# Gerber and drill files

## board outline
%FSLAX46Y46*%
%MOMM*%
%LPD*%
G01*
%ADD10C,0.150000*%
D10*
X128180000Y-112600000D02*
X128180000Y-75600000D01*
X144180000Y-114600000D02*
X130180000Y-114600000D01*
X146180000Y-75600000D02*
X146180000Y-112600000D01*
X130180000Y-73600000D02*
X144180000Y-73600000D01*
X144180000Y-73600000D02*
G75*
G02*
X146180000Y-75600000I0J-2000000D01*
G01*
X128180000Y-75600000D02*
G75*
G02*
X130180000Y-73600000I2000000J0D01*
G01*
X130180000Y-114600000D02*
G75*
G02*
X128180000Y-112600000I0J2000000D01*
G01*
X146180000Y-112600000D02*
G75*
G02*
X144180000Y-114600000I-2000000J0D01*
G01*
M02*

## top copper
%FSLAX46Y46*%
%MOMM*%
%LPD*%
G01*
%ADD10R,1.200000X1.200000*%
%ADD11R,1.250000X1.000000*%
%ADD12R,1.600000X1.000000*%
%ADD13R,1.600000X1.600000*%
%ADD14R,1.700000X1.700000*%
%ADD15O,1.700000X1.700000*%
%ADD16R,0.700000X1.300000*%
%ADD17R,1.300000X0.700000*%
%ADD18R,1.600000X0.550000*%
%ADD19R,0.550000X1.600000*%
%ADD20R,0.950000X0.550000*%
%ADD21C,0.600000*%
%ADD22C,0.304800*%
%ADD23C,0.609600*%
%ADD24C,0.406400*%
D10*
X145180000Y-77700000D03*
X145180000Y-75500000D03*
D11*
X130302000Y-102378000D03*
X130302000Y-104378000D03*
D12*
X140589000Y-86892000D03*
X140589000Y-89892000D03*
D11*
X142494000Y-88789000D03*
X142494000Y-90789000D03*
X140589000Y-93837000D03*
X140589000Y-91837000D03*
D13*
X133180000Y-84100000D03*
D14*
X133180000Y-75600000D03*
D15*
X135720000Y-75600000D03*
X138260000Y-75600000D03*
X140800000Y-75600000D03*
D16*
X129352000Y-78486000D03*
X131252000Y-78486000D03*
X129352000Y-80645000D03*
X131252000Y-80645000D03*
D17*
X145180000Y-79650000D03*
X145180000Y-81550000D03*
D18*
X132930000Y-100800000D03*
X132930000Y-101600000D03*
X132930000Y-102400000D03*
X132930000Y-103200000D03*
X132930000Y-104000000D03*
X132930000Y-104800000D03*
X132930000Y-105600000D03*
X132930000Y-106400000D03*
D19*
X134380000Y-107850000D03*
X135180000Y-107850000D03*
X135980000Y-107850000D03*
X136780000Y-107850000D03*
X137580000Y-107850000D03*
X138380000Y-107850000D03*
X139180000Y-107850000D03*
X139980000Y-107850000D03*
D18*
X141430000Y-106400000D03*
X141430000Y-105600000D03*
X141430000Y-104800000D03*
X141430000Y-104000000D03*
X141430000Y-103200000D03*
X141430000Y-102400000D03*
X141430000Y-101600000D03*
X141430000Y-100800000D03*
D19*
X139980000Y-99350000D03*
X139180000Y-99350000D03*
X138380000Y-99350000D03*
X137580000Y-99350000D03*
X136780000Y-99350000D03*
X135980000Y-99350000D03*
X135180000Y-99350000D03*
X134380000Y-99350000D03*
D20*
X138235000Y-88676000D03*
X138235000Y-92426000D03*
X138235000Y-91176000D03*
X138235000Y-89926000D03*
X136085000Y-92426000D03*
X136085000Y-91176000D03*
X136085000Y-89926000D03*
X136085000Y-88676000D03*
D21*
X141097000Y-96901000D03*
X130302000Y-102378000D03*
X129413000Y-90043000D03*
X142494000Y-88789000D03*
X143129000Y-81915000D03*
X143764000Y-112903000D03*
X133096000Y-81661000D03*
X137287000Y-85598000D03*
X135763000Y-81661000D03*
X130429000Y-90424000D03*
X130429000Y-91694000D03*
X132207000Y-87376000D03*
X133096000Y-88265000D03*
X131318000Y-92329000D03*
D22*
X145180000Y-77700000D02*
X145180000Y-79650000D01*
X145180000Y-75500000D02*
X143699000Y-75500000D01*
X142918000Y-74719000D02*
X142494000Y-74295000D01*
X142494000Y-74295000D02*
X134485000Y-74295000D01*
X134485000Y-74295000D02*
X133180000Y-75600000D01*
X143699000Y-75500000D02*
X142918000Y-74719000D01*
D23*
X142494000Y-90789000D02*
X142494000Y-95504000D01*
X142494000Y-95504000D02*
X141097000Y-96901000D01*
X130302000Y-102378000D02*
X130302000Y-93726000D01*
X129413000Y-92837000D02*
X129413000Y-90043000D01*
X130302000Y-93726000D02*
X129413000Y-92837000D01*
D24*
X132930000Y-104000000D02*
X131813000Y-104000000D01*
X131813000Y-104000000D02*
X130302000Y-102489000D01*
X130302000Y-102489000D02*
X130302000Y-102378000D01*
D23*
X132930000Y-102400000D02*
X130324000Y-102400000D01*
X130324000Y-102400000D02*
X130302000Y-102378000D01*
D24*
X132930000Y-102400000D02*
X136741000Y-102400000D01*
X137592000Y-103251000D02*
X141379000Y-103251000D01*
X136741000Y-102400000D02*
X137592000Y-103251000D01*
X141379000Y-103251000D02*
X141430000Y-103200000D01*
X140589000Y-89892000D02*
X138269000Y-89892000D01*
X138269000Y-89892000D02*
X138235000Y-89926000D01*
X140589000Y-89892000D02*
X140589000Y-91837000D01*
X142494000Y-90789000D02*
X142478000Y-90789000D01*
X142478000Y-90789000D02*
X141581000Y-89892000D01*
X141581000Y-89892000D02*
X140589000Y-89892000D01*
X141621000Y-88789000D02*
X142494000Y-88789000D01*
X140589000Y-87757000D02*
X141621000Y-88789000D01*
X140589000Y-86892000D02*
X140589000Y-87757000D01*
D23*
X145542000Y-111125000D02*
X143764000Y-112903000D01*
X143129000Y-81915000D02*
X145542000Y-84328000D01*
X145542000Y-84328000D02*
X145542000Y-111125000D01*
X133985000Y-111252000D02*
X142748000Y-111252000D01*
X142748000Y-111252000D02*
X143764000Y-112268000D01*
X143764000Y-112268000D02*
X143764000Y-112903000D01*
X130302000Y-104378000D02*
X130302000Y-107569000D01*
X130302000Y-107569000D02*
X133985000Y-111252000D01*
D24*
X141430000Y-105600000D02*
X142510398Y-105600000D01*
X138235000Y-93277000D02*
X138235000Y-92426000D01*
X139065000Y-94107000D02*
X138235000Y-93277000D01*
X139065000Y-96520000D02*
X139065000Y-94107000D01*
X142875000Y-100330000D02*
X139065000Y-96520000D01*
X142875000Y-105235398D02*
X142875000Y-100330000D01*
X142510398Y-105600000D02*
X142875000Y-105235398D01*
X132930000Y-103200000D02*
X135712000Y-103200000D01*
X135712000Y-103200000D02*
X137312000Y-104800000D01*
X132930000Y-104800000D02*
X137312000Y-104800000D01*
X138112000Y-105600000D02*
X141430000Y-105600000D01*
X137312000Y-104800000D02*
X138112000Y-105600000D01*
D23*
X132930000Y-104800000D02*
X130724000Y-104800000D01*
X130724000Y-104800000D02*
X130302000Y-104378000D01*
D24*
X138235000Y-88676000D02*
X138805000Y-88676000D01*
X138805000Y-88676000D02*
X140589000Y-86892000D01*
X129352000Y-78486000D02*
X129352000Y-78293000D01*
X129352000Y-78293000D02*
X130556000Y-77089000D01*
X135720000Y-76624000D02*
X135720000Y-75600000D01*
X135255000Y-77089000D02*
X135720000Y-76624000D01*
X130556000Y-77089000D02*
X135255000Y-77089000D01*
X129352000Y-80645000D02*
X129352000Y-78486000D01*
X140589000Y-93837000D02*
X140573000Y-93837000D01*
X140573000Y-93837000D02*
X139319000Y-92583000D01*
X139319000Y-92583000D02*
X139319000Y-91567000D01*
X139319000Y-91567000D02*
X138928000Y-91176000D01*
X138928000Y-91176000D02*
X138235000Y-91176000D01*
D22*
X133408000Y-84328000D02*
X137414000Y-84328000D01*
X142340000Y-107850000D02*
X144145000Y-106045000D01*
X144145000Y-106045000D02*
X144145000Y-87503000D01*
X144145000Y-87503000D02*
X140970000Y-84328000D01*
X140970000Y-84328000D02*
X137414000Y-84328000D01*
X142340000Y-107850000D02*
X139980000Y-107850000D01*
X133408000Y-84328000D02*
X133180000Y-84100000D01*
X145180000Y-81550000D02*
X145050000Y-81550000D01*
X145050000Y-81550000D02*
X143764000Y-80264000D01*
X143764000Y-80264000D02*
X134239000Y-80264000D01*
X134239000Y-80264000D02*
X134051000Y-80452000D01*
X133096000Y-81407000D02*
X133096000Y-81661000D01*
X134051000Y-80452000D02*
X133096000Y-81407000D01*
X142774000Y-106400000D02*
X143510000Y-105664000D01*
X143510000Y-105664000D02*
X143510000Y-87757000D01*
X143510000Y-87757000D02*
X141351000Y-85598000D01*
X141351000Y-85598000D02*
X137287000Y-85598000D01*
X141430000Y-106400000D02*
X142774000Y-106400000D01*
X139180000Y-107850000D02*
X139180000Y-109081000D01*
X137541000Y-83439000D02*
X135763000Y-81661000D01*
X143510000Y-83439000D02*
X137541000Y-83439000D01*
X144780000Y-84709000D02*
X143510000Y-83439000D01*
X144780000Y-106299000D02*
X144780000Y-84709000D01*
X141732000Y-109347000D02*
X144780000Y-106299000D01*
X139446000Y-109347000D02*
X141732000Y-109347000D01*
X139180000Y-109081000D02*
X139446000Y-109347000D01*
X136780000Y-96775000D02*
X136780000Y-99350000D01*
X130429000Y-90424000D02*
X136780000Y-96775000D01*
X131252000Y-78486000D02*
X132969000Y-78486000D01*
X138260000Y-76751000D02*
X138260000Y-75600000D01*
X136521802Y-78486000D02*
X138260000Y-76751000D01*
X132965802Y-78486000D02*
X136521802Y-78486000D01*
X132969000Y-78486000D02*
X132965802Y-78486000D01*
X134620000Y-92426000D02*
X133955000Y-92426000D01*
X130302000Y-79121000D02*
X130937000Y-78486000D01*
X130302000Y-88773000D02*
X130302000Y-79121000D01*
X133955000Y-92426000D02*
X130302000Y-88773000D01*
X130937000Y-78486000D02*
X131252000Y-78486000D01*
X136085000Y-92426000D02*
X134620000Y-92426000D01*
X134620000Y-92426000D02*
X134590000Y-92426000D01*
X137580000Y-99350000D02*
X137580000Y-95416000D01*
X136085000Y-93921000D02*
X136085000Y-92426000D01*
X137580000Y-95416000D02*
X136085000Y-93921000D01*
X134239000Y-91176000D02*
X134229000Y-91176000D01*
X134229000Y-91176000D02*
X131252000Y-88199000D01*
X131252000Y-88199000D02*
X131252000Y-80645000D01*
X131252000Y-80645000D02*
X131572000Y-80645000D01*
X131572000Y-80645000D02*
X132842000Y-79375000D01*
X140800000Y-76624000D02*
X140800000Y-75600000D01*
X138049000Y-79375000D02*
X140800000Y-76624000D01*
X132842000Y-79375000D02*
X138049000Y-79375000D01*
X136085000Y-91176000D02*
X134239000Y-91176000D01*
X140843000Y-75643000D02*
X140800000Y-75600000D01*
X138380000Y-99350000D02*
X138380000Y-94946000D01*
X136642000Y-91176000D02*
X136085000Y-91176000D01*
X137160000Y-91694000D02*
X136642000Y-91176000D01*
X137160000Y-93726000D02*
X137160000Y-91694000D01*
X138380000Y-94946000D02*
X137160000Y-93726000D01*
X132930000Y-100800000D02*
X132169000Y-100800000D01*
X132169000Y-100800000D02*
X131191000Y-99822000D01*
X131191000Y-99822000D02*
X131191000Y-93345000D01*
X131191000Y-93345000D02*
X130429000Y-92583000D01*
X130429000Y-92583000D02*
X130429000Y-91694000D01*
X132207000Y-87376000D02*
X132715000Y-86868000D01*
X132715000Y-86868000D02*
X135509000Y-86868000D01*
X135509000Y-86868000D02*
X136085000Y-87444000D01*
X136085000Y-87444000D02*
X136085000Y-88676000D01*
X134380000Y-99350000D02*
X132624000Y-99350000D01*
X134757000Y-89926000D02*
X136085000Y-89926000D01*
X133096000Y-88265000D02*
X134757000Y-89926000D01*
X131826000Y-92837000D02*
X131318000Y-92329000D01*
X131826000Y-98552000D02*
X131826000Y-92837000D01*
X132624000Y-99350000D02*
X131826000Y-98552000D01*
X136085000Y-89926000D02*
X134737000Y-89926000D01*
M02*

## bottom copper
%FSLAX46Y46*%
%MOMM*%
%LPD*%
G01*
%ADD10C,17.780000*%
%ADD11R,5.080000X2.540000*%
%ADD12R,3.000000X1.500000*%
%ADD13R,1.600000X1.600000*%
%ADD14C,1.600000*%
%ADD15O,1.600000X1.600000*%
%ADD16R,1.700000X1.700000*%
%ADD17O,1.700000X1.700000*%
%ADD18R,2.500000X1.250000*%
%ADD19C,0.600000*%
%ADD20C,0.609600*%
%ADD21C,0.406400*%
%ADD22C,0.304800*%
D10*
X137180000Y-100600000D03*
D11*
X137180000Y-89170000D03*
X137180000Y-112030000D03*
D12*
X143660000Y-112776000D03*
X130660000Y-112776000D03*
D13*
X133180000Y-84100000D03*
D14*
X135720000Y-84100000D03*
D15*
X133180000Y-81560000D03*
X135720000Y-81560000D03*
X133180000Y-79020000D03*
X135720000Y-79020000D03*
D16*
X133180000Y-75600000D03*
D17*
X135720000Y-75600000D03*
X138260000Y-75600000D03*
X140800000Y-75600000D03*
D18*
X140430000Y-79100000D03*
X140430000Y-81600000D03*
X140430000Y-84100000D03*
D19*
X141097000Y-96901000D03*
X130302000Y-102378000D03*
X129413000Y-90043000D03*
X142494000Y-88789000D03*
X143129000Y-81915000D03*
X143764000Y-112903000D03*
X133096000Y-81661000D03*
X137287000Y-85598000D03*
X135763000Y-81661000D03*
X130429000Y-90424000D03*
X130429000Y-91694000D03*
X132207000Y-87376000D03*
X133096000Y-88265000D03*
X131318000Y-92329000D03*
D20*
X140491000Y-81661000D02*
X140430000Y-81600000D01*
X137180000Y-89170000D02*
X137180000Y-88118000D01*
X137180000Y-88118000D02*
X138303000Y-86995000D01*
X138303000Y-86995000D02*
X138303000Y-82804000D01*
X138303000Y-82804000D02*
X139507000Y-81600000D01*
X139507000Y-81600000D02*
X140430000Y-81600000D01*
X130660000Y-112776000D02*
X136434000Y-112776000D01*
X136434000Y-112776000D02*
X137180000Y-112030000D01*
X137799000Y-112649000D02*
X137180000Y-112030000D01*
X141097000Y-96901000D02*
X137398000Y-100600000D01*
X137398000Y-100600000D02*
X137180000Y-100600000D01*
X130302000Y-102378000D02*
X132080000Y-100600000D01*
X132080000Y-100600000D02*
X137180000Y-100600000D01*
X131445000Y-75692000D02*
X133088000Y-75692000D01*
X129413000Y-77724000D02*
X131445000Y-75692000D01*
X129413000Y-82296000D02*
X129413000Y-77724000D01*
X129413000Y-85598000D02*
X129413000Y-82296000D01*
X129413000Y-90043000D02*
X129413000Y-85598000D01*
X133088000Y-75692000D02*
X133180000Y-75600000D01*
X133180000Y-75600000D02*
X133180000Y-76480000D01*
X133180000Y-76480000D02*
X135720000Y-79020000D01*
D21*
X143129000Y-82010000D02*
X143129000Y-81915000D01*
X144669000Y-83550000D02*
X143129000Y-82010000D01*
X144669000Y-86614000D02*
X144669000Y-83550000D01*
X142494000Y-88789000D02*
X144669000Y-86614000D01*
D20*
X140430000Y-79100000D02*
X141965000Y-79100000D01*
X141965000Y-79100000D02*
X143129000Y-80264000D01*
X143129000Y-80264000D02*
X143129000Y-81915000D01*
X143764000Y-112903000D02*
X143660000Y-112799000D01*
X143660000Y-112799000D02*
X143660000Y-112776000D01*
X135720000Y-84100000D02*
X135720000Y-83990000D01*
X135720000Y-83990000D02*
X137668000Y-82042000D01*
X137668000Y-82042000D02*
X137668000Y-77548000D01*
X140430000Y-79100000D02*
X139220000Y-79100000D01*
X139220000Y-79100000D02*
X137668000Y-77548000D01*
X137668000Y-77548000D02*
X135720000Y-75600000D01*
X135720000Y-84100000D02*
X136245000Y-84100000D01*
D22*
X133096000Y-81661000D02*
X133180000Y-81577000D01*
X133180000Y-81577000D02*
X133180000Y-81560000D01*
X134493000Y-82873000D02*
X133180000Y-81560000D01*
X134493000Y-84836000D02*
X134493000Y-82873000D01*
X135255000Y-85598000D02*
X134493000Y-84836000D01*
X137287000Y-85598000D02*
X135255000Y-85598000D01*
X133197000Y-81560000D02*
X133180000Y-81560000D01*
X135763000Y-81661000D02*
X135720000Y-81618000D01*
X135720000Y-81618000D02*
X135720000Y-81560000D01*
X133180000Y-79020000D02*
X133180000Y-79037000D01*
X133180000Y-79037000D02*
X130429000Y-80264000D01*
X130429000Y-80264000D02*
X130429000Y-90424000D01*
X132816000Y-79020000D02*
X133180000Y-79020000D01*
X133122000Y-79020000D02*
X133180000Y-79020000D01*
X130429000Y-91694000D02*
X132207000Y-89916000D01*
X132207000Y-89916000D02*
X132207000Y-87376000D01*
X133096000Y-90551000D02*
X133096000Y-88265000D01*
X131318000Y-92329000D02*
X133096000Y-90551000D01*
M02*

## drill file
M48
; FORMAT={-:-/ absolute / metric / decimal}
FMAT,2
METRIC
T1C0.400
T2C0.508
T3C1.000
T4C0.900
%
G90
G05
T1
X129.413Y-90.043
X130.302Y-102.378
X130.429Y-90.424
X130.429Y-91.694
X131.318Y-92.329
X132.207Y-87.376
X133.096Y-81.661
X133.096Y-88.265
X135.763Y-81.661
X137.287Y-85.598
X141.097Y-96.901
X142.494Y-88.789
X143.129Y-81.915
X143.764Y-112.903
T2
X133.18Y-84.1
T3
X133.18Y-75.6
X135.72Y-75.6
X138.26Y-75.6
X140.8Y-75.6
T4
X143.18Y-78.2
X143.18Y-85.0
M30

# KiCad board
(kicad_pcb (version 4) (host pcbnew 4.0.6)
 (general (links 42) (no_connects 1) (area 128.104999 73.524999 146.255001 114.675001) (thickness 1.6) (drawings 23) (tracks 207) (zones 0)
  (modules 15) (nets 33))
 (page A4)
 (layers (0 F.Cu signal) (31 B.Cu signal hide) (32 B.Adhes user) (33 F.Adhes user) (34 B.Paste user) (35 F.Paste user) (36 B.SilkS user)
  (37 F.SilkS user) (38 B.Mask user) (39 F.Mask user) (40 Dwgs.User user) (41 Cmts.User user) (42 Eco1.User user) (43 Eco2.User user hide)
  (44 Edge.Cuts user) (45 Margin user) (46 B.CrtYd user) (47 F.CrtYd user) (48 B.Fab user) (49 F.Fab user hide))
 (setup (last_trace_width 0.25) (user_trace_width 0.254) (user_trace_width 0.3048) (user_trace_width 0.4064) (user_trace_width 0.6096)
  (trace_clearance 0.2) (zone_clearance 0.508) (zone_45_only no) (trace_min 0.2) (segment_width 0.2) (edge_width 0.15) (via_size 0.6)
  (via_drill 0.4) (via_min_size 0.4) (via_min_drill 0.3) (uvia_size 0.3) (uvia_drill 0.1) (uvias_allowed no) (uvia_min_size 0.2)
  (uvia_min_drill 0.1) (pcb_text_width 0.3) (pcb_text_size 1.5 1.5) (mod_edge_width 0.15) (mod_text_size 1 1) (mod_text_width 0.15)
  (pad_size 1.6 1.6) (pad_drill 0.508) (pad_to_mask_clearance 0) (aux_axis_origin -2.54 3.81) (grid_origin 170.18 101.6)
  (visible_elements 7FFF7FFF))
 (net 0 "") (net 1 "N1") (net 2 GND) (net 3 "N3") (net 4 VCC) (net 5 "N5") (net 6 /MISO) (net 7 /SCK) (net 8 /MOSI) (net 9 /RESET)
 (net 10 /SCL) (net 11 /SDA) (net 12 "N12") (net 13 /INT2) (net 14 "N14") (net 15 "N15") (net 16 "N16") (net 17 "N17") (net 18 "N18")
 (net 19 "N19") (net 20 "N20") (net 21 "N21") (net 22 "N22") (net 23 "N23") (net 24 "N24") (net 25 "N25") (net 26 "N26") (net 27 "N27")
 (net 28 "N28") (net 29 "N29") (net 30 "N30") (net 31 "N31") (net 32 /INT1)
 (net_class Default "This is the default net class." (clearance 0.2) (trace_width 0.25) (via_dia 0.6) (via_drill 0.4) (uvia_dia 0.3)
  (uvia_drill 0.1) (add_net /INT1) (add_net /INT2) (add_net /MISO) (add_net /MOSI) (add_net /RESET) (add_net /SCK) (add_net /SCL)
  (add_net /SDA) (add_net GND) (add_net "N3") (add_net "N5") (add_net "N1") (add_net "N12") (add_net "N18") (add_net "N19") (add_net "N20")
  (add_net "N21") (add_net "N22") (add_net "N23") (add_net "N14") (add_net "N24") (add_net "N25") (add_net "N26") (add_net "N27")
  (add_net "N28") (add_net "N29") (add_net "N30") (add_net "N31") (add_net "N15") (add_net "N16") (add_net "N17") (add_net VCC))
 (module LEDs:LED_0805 (layer F.Cu) (at 145.18 76.6 270)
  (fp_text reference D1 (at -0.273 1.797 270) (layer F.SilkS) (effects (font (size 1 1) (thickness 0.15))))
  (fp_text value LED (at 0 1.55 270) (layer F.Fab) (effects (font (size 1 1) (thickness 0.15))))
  (pad 2 smd rect (at 1.1 0 90) (size 1.2 1.2) (layers F.Cu F.Paste F.Mask) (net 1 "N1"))
  (pad 1 smd rect (at -1.1 0 90) (size 1.2 1.2) (layers F.Cu F.Paste F.Mask) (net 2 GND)))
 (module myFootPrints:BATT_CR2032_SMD (layer B.Cu) (at 137.18 100.6 270)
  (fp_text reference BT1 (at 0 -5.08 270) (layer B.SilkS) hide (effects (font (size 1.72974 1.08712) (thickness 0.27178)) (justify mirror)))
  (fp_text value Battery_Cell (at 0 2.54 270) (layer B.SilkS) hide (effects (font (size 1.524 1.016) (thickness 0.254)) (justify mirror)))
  (pad 2 smd circle (at 0 0 270) (size 17.78 17.78) (layers B.Cu B.Paste B.Mask) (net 2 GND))
  (pad 1 smd rect (at -11.43 0 270) (size 2.54 5.08) (layers B.Cu B.Paste B.Mask) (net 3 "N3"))
  (pad 1 smd rect (at 11.43 0 270) (size 2.54 5.08) (layers B.Cu B.Paste B.Mask) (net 3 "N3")))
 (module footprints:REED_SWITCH (layer B.Cu) (at 137.16 112.776 180)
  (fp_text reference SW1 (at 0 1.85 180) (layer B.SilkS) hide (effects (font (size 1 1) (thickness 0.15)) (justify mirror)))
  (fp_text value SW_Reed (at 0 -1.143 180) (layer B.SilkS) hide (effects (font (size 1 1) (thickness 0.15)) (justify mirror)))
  (pad 1 smd rect (at -6.5 0 180) (size 3 1.5) (layers B.Cu B.Paste B.Mask) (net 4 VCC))
  (pad 2 smd rect (at 6.5 0 180) (size 3 1.5) (layers B.Cu B.Paste B.Mask) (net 3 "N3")))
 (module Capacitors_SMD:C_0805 (layer F.Cu) (at 130.302 103.378 270)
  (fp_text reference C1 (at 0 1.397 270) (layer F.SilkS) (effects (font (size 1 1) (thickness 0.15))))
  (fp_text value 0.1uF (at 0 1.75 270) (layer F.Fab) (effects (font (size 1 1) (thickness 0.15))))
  (pad 1 smd rect (at -1 0 270) (size 1 1.25) (layers F.Cu F.Paste F.Mask) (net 2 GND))
  (pad 2 smd rect (at 1 0 270) (size 1 1.25) (layers F.Cu F.Paste F.Mask) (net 4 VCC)))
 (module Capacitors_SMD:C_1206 (layer F.Cu) (at 140.589 88.392 270)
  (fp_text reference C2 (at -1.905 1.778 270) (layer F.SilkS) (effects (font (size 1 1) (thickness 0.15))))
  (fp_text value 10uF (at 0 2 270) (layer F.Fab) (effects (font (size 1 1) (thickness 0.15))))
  (pad 1 smd rect (at -1.5 0 270) (size 1 1.6) (layers F.Cu F.Paste F.Mask) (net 4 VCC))
  (pad 2 smd rect (at 1.5 0 270) (size 1 1.6) (layers F.Cu F.Paste F.Mask) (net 2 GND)))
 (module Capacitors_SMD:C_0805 (layer F.Cu) (at 142.494 89.789 270)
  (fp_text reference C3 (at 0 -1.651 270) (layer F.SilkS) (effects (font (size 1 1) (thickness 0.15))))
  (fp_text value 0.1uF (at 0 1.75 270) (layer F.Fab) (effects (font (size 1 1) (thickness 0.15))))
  (pad 1 smd rect (at -1 0 270) (size 1 1.25) (layers F.Cu F.Paste F.Mask) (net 4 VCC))
  (pad 2 smd rect (at 1 0 270) (size 1 1.25) (layers F.Cu F.Paste F.Mask) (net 2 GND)))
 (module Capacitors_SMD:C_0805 (layer F.Cu) (at 140.589 92.837 90)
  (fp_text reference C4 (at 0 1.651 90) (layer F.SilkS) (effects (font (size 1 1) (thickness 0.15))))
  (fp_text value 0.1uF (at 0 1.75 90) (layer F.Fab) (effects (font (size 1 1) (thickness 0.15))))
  (pad 1 smd rect (at -1 0 90) (size 1 1.25) (layers F.Cu F.Paste F.Mask) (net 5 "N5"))
  (pad 2 smd rect (at 1 0 90) (size 1 1.25) (layers F.Cu F.Paste F.Mask) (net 2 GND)))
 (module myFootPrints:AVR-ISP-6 (layer B.Cu) (at 133.18 84.1)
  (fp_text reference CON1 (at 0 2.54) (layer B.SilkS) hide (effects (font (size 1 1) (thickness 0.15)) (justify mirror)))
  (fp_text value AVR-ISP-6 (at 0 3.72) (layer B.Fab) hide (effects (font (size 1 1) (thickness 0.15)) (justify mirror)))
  (pad 1 thru_hole rect (at 0 0) (size 1.6 1.6) (drill 0.508) (layers *.Cu B.Mask) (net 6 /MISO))
  (pad 2 smd circle (at 2.54 0) (size 1.6 1.6) (layers B.Cu B.Paste B.Mask) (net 4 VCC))
  (pad 3 smd oval (at 0 -2.54) (size 1.6 1.6) (layers B.Cu B.Paste B.Mask) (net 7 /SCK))
  (pad 4 smd oval (at 2.54 -2.54) (size 1.6 1.6) (layers B.Cu B.Paste B.Mask) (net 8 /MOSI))
  (pad 5 smd oval (at 0 -5.08) (size 1.6 1.6) (layers B.Cu B.Paste B.Mask) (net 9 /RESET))
  (pad 6 smd oval (at 2.54 -5.08) (size 1.6 1.6) (layers B.Cu B.Paste B.Mask) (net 2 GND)))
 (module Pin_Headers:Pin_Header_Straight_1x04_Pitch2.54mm (layer F.Cu) (at 133.18 75.6 90)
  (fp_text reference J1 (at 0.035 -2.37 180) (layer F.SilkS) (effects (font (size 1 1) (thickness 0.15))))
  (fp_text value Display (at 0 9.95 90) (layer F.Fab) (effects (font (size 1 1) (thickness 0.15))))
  (pad 1 thru_hole rect (at 0 0 90) (size 1.7 1.7) (drill 1) (layers *.Cu *.Mask) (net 2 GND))
  (pad 2 thru_hole oval (at 0 2.54 90) (size 1.7 1.7) (drill 1) (layers *.Cu *.Mask) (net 4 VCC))
  (pad 3 thru_hole oval (at 0 5.08 90) (size 1.7 1.7) (drill 1) (layers *.Cu *.Mask) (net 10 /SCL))
  (pad 4 thru_hole oval (at 0 7.62 90) (size 1.7 1.7) (drill 1) (layers *.Cu *.Mask) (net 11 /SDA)))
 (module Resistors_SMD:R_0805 (layer F.Cu) (at 130.302 78.486)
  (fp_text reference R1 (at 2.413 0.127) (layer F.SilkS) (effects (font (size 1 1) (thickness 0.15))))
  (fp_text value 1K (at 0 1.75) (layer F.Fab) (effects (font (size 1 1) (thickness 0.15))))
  (pad 1 smd rect (at -0.95 0) (size 0.7 1.3) (layers F.Cu F.Paste F.Mask) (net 4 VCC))
  (pad 2 smd rect (at 0.95 0) (size 0.7 1.3) (layers F.Cu F.Paste F.Mask) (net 10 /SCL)))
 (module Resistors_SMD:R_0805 (layer F.Cu) (at 130.302 80.645)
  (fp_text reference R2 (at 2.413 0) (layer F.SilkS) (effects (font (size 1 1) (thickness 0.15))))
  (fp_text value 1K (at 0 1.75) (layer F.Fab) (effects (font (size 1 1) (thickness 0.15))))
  (pad 1 smd rect (at -0.95 0) (size 0.7 1.3) (layers F.Cu F.Paste F.Mask) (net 4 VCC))
  (pad 2 smd rect (at 0.95 0) (size 0.7 1.3) (layers F.Cu F.Paste F.Mask) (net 11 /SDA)))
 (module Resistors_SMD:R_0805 (layer F.Cu) (at 145.18 80.6 270)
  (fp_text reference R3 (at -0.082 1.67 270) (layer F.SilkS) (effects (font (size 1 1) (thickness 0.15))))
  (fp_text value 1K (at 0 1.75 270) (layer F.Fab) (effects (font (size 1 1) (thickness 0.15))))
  (pad 1 smd rect (at -0.95 0 270) (size 0.7 1.3) (layers F.Cu F.Paste F.Mask) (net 1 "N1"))
  (pad 2 smd rect (at 0.95 0 270) (size 0.7 1.3) (layers F.Cu F.Paste F.Mask) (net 7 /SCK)))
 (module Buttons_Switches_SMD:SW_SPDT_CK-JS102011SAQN (layer B.Cu) (at 143.18 81.6 270)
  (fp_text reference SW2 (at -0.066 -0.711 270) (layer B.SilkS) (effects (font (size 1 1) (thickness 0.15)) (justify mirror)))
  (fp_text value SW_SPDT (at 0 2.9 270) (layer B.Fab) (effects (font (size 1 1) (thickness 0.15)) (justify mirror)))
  (pad 1 smd rect (at -2.5 2.75 270) (size 1.25 2.5) (layers B.Cu B.Paste B.Mask) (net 4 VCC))
  (pad 2 smd rect (at 0 2.75 270) (size 1.25 2.5) (layers B.Cu B.Paste B.Mask) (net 3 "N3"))
  (pad 3 smd rect (at 2.5 2.75 270) (size 1.25 2.5) (layers B.Cu B.Paste B.Mask) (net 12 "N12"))
  (pad "" np_thru_hole circle (at -3.4 0 270) (size 0.9 0.9) (drill 0.9) (layers *.Cu *.Mask))
  (pad "" np_thru_hole circle (at 3.4 0 270) (size 0.9 0.9) (drill 0.9) (layers *.Cu *.Mask)))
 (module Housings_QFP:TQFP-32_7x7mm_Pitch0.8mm (layer F.Cu) (at 137.18 103.6)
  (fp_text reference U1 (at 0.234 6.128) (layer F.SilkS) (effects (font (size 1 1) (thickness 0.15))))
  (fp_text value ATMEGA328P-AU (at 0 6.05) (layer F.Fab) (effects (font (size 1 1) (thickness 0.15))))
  (pad 1 smd rect (at -4.25 -2.8) (size 1.6 0.55) (layers F.Cu F.Paste F.Mask) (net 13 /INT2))
  (pad 2 smd rect (at -4.25 -2) (size 1.6 0.55) (layers F.Cu F.Paste F.Mask) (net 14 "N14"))
  (pad 3 smd rect (at -4.25 -1.2) (size 1.6 0.55) (layers F.Cu F.Paste F.Mask) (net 2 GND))
  (pad 4 smd rect (at -4.25 -0.4) (size 1.6 0.55) (layers F.Cu F.Paste F.Mask) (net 4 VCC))
  (pad 5 smd rect (at -4.25 0.4) (size 1.6 0.55) (layers F.Cu F.Paste F.Mask) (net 2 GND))
  (pad 6 smd rect (at -4.25 1.2) (size 1.6 0.55) (layers F.Cu F.Paste F.Mask) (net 4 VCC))
  (pad 7 smd rect (at -4.25 2) (size 1.6 0.55) (layers F.Cu F.Paste F.Mask) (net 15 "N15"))
  (pad 8 smd rect (at -4.25 2.8) (size 1.6 0.55) (layers F.Cu F.Paste F.Mask) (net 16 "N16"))
  (pad 9 smd rect (at -2.8 4.25 90) (size 1.6 0.55) (layers F.Cu F.Paste F.Mask) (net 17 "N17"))
  (pad 10 smd rect (at -2 4.25 90) (size 1.6 0.55) (layers F.Cu F.Paste F.Mask) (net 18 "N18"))
  (pad 11 smd rect (at -1.2 4.25 90) (size 1.6 0.55) (layers F.Cu F.Paste F.Mask) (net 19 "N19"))
  (pad 12 smd rect (at -0.4 4.25 90) (size 1.6 0.55) (layers F.Cu F.Paste F.Mask) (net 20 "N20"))
  (pad 13 smd rect (at 0.4 4.25 90) (size 1.6 0.55) (layers F.Cu F.Paste F.Mask) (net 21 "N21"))
  (pad 14 smd rect (at 1.2 4.25 90) (size 1.6 0.55) (layers F.Cu F.Paste F.Mask) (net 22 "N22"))
  (pad 15 smd rect (at 2 4.25 90) (size 1.6 0.55) (layers F.Cu F.Paste F.Mask) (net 8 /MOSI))
  (pad 16 smd rect (at 2.8 4.25 90) (size 1.6 0.55) (layers F.Cu F.Paste F.Mask) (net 6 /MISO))
  (pad 17 smd rect (at 4.25 2.8) (size 1.6 0.55) (layers F.Cu F.Paste F.Mask) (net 7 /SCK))
  (pad 18 smd rect (at 4.25 2) (size 1.6 0.55) (layers F.Cu F.Paste F.Mask) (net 4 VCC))
  (pad 19 smd rect (at 4.25 1.2) (size 1.6 0.55) (layers F.Cu F.Paste F.Mask) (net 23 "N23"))
  (pad 20 smd rect (at 4.25 0.4) (size 1.6 0.55) (layers F.Cu F.Paste F.Mask) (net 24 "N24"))
  (pad 21 smd rect (at 4.25 -0.4) (size 1.6 0.55) (layers F.Cu F.Paste F.Mask) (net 2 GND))
  (pad 22 smd rect (at 4.25 -1.2) (size 1.6 0.55) (layers F.Cu F.Paste F.Mask) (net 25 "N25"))
  (pad 23 smd rect (at 4.25 -2) (size 1.6 0.55) (layers F.Cu F.Paste F.Mask) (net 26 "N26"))
  (pad 24 smd rect (at 4.25 -2.8) (size 1.6 0.55) (layers F.Cu F.Paste F.Mask) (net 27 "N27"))
  (pad 25 smd rect (at 2.8 -4.25 90) (size 1.6 0.55) (layers F.Cu F.Paste F.Mask) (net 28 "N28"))
  (pad 26 smd rect (at 2 -4.25 90) (size 1.6 0.55) (layers F.Cu F.Paste F.Mask) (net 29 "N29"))
  (pad 27 smd rect (at 1.2 -4.25 90) (size 1.6 0.55) (layers F.Cu F.Paste F.Mask) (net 11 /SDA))
  (pad 28 smd rect (at 0.4 -4.25 90) (size 1.6 0.55) (layers F.Cu F.Paste F.Mask) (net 10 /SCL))
  (pad 29 smd rect (at -0.4 -4.25 90) (size 1.6 0.55) (layers F.Cu F.Paste F.Mask) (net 9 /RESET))
  (pad 30 smd rect (at -1.2 -4.25 90) (size 1.6 0.55) (layers F.Cu F.Paste F.Mask) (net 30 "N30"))
  (pad 31 smd rect (at -2 -4.25 90) (size 1.6 0.55) (layers F.Cu F.Paste F.Mask) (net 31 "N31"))
  (pad 32 smd rect (at -2.8 -4.25 90) (size 1.6 0.55) (layers F.Cu F.Paste F.Mask) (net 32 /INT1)))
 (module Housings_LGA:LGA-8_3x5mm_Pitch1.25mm (layer F.Cu) (at 137.16 90.551 180)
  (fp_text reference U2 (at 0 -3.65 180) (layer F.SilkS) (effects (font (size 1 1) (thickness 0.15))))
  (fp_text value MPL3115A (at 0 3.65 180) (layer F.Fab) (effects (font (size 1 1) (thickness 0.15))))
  (pad 4 smd rect (at -1.075 1.875 180) (size 0.95 0.55) (layers F.Cu F.Paste F.Mask) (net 4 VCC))
  (pad 1 smd rect (at -1.075 -1.875 180) (size 0.95 0.55) (layers F.Cu F.Paste F.Mask) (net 4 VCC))
  (pad 2 smd rect (at -1.075 -0.625 180) (size 0.95 0.55) (layers F.Cu F.Paste F.Mask) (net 5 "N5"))
  (pad 3 smd rect (at -1.075 0.625 180) (size 0.95 0.55) (layers F.Cu F.Paste F.Mask) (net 2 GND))
  (pad 8 smd rect (at 1.075 -1.875 180) (size 0.95 0.55) (layers F.Cu F.Paste F.Mask) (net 10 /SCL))
  (pad 7 smd rect (at 1.075 -0.625 180) (size 0.95 0.55) (layers F.Cu F.Paste F.Mask) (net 11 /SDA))
  (pad 6 smd rect (at 1.075 0.625 180) (size 0.95 0.55) (layers F.Cu F.Paste F.Mask) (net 32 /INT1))
  (pad 5 smd rect (at 1.075 1.875 180) (size 0.95 0.55) (layers F.Cu F.Paste F.Mask) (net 13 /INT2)))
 (gr_line (start 128.18 112.6) (end 128.18 75.6) (angle 90) (layer Edge.Cuts) (width 0.15))
 (gr_line (start 144.18 114.6) (end 130.18 114.6) (angle 90) (layer Edge.Cuts) (width 0.15))
 (gr_line (start 146.18 75.6) (end 146.18 112.6) (angle 90) (layer Edge.Cuts) (width 0.15))
 (gr_line (start 130.18 73.6) (end 144.18 73.6) (angle 90) (layer Edge.Cuts) (width 0.15))
 (gr_arc (start 144.18 75.6) (end 144.18 73.6) (angle 90) (layer Edge.Cuts) (width 0.15))
 (gr_arc (start 130.18 75.6) (end 128.18 75.6) (angle 90) (layer Edge.Cuts) (width 0.15))
 (gr_arc (start 130.18 112.6) (end 130.18 114.6) (angle 90) (layer Edge.Cuts) (width 0.15))
 (gr_arc (start 144.18 112.6) (end 146.18 112.6) (angle 90) (layer Edge.Cuts) (width 0.15))
 (segment (start 140.491 81.661) (end 140.43 81.6) (width 0.6096) (layer B.Cu) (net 3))
 (segment (start 137.18 89.17) (end 137.18 88.118) (width 0.6096) (layer B.Cu) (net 3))
 (segment (start 137.18 88.118) (end 138.303 86.995) (width 0.6096) (layer B.Cu) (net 3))
 (segment (start 138.303 86.995) (end 138.303 82.804) (width 0.6096) (layer B.Cu) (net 3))
 (segment (start 138.303 82.804) (end 139.507 81.6) (width 0.6096) (layer B.Cu) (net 3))
 (segment (start 139.507 81.6) (end 140.43 81.6) (width 0.6096) (layer B.Cu) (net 3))
 (segment (start 130.66 112.776) (end 136.434 112.776) (width 0.6096) (layer B.Cu) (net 3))
 (segment (start 136.434 112.776) (end 137.18 112.03) (width 0.6096) (layer B.Cu) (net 3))
 (segment (start 137.799 112.649) (end 137.18 112.03) (width 0.6096) (layer B.Cu) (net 3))
 (segment (start 145.18 77.7) (end 145.18 79.65) (width 0.3048) (layer F.Cu) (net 1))
 (segment (start 145.18 75.5) (end 143.699 75.5) (width 0.3048) (layer F.Cu) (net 2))
 (segment (start 142.918 74.719) (end 142.494 74.295) (width 0.3048) (layer F.Cu) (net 2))
 (segment (start 142.494 74.295) (end 134.485 74.295) (width 0.3048) (layer F.Cu) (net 2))
 (segment (start 134.485 74.295) (end 133.18 75.6) (width 0.3048) (layer F.Cu) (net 2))
 (segment (start 143.699 75.5) (end 142.918 74.719) (width 0.3048) (layer F.Cu) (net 2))
 (segment (start 142.494 90.789) (end 142.494 95.504) (width 0.6096) (layer F.Cu) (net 2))
 (segment (start 141.097 96.901) (end 137.398 100.6) (width 0.6096) (layer B.Cu) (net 2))
 (via (at 141.097 96.901) (size 0.6) (drill 0.4) (layers F.Cu B.Cu) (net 2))
 (segment (start 142.494 95.504) (end 141.097 96.901) (width 0.6096) (layer F.Cu) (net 2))
 (segment (start 137.398 100.6) (end 137.18 100.6) (width 0.6096) (layer B.Cu) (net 2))
 (via (at 130.302 102.378) (size 0.6) (drill 0.4) (layers F.Cu B.Cu) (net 2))
 (segment (start 130.302 102.378) (end 132.08 100.6) (width 0.6096) (layer B.Cu) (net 2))
 (segment (start 132.08 100.6) (end 137.18 100.6) (width 0.6096) (layer B.Cu) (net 2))
 (segment (start 130.302 102.378) (end 130.302 93.726) (width 0.6096) (layer F.Cu) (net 2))
 (segment (start 131.445 75.692) (end 133.088 75.692) (width 0.6096) (layer B.Cu) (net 2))
 (segment (start 129.413 77.724) (end 131.445 75.692) (width 0.6096) (layer B.Cu) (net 2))
 (segment (start 129.413 82.296) (end 129.413 77.724) (width 0.6096) (layer B.Cu) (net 2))
 (segment (start 129.413 85.598) (end 129.413 82.296) (width 0.6096) (layer B.Cu) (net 2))
 (segment (start 129.413 90.043) (end 129.413 85.598) (width 0.6096) (layer B.Cu) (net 2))
 (via (at 129.413 90.043) (size 0.6) (drill 0.4) (layers F.Cu B.Cu) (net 2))
 (segment (start 129.413 92.837) (end 129.413 90.043) (width 0.6096) (layer F.Cu) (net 2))
 (segment (start 130.302 93.726) (end 129.413 92.837) (width 0.6096) (layer F.Cu) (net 2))
 (segment (start 133.088 75.692) (end 133.18 75.6) (width 0.6096) (layer B.Cu) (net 2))
 (segment (start 132.93 104) (end 131.813 104) (width 0.4064) (layer F.Cu) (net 2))
 (segment (start 131.813 104) (end 130.302 102.489) (width 0.4064) (layer F.Cu) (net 2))
 (segment (start 130.302 102.489) (end 130.302 102.378) (width 0.4064) (layer F.Cu) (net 2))
 (segment (start 132.93 102.4) (end 130.324 102.4) (width 0.6096) (layer F.Cu) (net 2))
 (segment (start 130.324 102.4) (end 130.302 102.378) (width 0.6096) (layer F.Cu) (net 2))
 (segment (start 132.93 102.4) (end 136.741 102.4) (width 0.4064) (layer F.Cu) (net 2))
 (segment (start 137.592 103.251) (end 141.379 103.251) (width 0.4064) (layer F.Cu) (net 2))
 (segment (start 136.741 102.4) (end 137.592 103.251) (width 0.4064) (layer F.Cu) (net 2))
 (segment (start 141.379 103.251) (end 141.43 103.2) (width 0.4064) (layer F.Cu) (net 2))
 (segment (start 140.589 89.892) (end 138.269 89.892) (width 0.4064) (layer F.Cu) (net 2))
 (segment (start 138.269 89.892) (end 138.235 89.926) (width 0.4064) (layer F.Cu) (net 2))
 (segment (start 140.589 89.892) (end 140.589 91.837) (width 0.4064) (layer F.Cu) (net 2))
 (segment (start 142.494 90.789) (end 142.478 90.789) (width 0.4064) (layer F.Cu) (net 2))
 (segment (start 142.478 90.789) (end 141.581 89.892) (width 0.4064) (layer F.Cu) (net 2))
 (segment (start 141.581 89.892) (end 140.589 89.892) (width 0.4064) (layer F.Cu) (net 2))
 (segment (start 133.18 75.6) (end 133.18 76.48) (width 0.6096) (layer B.Cu) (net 2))
 (segment (start 133.18 76.48) (end 135.72 79.02) (width 0.6096) (layer B.Cu) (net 2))
 (via (at 142.494 88.789) (size 0.6) (drill 0.4) (layers F.Cu B.Cu) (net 4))
 (segment (start 141.621 88.789) (end 142.494 88.789) (width 0.4064) (layer F.Cu) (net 4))
 (segment (start 140.589 87.757) (end 141.621 88.789) (width 0.4064) (layer F.Cu) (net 4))
 (segment (start 140.589 86.892) (end 140.589 87.757) (width 0.4064) (layer F.Cu) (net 4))
 (segment (start 143.129 82.01) (end 143.129 81.915) (width 0.4064) (layer B.Cu) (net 4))
 (segment (start 144.669 83.55) (end 143.129 82.01) (width 0.4064) (layer B.Cu) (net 4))
 (segment (start 144.669 86.614) (end 144.669 83.55) (width 0.4064) (layer B.Cu) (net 4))
 (segment (start 142.494 88.789) (end 144.669 86.614) (width 0.4064) (layer B.Cu) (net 4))
 (segment (start 140.43 79.1) (end 141.965 79.1) (width 0.6096) (layer B.Cu) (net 4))
 (segment (start 141.965 79.1) (end 143.129 80.264) (width 0.6096) (layer B.Cu) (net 4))
 (segment (start 143.129 80.264) (end 143.129 81.915) (width 0.6096) (layer B.Cu) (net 4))
 (segment (start 145.542 111.125) (end 143.764 112.903) (width 0.6096) (layer F.Cu) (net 4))
 (via (at 143.129 81.915) (size 0.6) (drill 0.4) (layers F.Cu B.Cu) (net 4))
 (segment (start 143.129 81.915) (end 145.542 84.328) (width 0.6096) (layer F.Cu) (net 4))
 (segment (start 145.542 84.328) (end 145.542 111.125) (width 0.6096) (layer F.Cu) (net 4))
 (segment (start 133.985 111.252) (end 142.748 111.252) (width 0.6096) (layer F.Cu) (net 4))
 (segment (start 142.748 111.252) (end 143.764 112.268) (width 0.6096) (layer F.Cu) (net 4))
 (segment (start 143.764 112.268) (end 143.764 112.903) (width 0.6096) (layer F.Cu) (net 4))
 (segment (start 130.302 104.378) (end 130.302 107.569) (width 0.6096) (layer F.Cu) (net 4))
 (segment (start 130.302 107.569) (end 133.985 111.252) (width 0.6096) (layer F.Cu) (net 4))
 (segment (start 143.764 112.903) (end 143.66 112.799) (width 0.6096) (layer B.Cu) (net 4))
 (via (at 143.764 112.903) (size 0.6) (drill 0.4) (layers F.Cu B.Cu) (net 4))
 (segment (start 143.66 112.799) (end 143.66 112.776) (width 0.6096) (layer B.Cu) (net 4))
 (segment (start 135.72 84.1) (end 135.72 83.99) (width 0.6096) (layer B.Cu) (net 4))
 (segment (start 135.72 83.99) (end 137.668 82.042) (width 0.6096) (layer B.Cu) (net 4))
 (segment (start 137.668 82.042) (end 137.668 77.548) (width 0.6096) (layer B.Cu) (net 4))
 (segment (start 140.43 79.1) (end 139.22 79.1) (width 0.6096) (layer B.Cu) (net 4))
 (segment (start 139.22 79.1) (end 137.668 77.548) (width 0.6096) (layer B.Cu) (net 4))
 (segment (start 137.668 77.548) (end 135.72 75.6) (width 0.6096) (layer B.Cu) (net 4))
 (segment (start 141.43 105.6) (end 142.510398 105.6) (width 0.4064) (layer F.Cu) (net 4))
 (segment (start 138.235 93.277) (end 138.235 92.426) (width 0.4064) (layer F.Cu) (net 4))
 (segment (start 139.065 94.107) (end 138.235 93.277) (width 0.4064) (layer F.Cu) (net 4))
 (segment (start 139.065 96.52) (end 139.065 94.107) (width 0.4064) (layer F.Cu) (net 4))
 (segment (start 142.875 100.33) (end 139.065 96.52) (width 0.4064) (layer F.Cu) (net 4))
 (segment (start 142.875 105.235398) (end 142.875 100.33) (width 0.4064) (layer F.Cu) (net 4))
 (segment (start 142.510398 105.6) (end 142.875 105.235398) (width 0.4064) (layer F.Cu) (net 4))
 (segment (start 132.93 103.2) (end 135.712 103.2) (width 0.4064) (layer F.Cu) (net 4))
 (segment (start 135.712 103.2) (end 137.312 104.8) (width 0.4064) (layer F.Cu) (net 4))
 (segment (start 132.93 104.8) (end 137.312 104.8) (width 0.4064) (layer F.Cu) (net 4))
 (segment (start 138.112 105.6) (end 141.43 105.6) (width 0.4064) (layer F.Cu) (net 4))
 (segment (start 137.312 104.8) (end 138.112 105.6) (width 0.4064) (layer F.Cu) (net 4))
 (segment (start 132.93 104.8) (end 130.724 104.8) (width 0.6096) (layer F.Cu) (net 4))
 (segment (start 130.724 104.8) (end 130.302 104.378) (width 0.6096) (layer F.Cu) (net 4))
 (segment (start 138.235 88.676) (end 138.805 88.676) (width 0.4064) (layer F.Cu) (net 4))
 (segment (start 138.805 88.676) (end 140.589 86.892) (width 0.4064) (layer F.Cu) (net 4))
 (segment (start 129.352 78.486) (end 129.352 78.293) (width 0.4064) (layer F.Cu) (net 4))
 (segment (start 129.352 78.293) (end 130.556 77.089) (width 0.4064) (layer F.Cu) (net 4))
 (segment (start 135.72 76.624) (end 135.72 75.6) (width 0.4064) (layer F.Cu) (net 4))
 (segment (start 135.255 77.089) (end 135.72 76.624) (width 0.4064) (layer F.Cu) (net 4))
 (segment (start 130.556 77.089) (end 135.255 77.089) (width 0.4064) (layer F.Cu) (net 4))
 (segment (start 129.352 80.645) (end 129.352 78.486) (width 0.4064) (layer F.Cu) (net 4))
 (segment (start 135.72 84.1) (end 136.245 84.1) (width 0.6096) (layer B.Cu) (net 4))
 (segment (start 140.589 93.837) (end 140.573 93.837) (width 0.4064) (layer F.Cu) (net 5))
 (segment (start 140.573 93.837) (end 139.319 92.583) (width 0.4064) (layer F.Cu) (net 5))
 (segment (start 139.319 92.583) (end 139.319 91.567) (width 0.4064) (layer F.Cu) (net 5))
 (segment (start 139.319 91.567) (end 138.928 91.176) (width 0.4064) (layer F.Cu) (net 5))
 (segment (start 138.928 91.176) (end 138.235 91.176) (width 0.4064) (layer F.Cu) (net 5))
 (segment (start 133.408 84.328) (end 137.414 84.328) (width 0.3048) (layer F.Cu) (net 6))
 (segment (start 142.34 107.85) (end 144.145 106.045) (width 0.3048) (layer F.Cu) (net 6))
 (segment (start 144.145 106.045) (end 144.145 87.503) (width 0.3048) (layer F.Cu) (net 6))
 (segment (start 144.145 87.503) (end 140.97 84.328) (width 0.3048) (layer F.Cu) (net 6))
 (segment (start 140.97 84.328) (end 137.414 84.328) (width 0.3048) (layer F.Cu) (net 6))
 (segment (start 142.34 107.85) (end 139.98 107.85) (width 0.3048) (layer F.Cu) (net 6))
 (segment (start 133.408 84.328) (end 133.18 84.1) (width 0.3048) (layer F.Cu) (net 6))
 (segment (start 145.18 81.55) (end 145.05 81.55) (width 0.3048) (layer F.Cu) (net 7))
 (segment (start 145.05 81.55) (end 143.764 80.264) (width 0.3048) (layer F.Cu) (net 7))
 (segment (start 143.764 80.264) (end 134.239 80.264) (width 0.3048) (layer F.Cu) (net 7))
 (segment (start 134.239 80.264) (end 134.051 80.452) (width 0.3048) (layer F.Cu) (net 7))
 (segment (start 133.096 81.661) (end 133.18 81.577) (width 0.3048) (layer B.Cu) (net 7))
 (via (at 133.096 81.661) (size 0.6) (drill 0.4) (layers F.Cu B.Cu) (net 7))
 (segment (start 133.096 81.407) (end 133.096 81.661) (width 0.3048) (layer F.Cu) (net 7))
 (segment (start 134.051 80.452) (end 133.096 81.407) (width 0.3048) (layer F.Cu) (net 7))
 (segment (start 133.18 81.577) (end 133.18 81.56) (width 0.3048) (layer B.Cu) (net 7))
 (via (at 137.287 85.598) (size 0.6) (drill 0.4) (layers F.Cu B.Cu) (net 7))
 (segment (start 142.774 106.4) (end 143.51 105.664) (width 0.3048) (layer F.Cu) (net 7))
 (segment (start 143.51 105.664) (end 143.51 87.757) (width 0.3048) (layer F.Cu) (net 7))
 (segment (start 143.51 87.757) (end 141.351 85.598) (width 0.3048) (layer F.Cu) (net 7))
 (segment (start 141.351 85.598) (end 137.287 85.598) (width 0.3048) (layer F.Cu) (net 7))
 (segment (start 141.43 106.4) (end 142.774 106.4) (width 0.3048) (layer F.Cu) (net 7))
 (segment (start 134.493 82.873) (end 133.18 81.56) (width 0.3048) (layer B.Cu) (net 7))
 (segment (start 134.493 84.836) (end 134.493 82.873) (width 0.3048) (layer B.Cu) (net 7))
 (segment (start 135.255 85.598) (end 134.493 84.836) (width 0.3048) (layer B.Cu) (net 7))
 (segment (start 137.287 85.598) (end 135.255 85.598) (width 0.3048) (layer B.Cu) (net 7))
 (segment (start 133.197 81.56) (end 133.18 81.56) (width 0.3048) (layer B.Cu) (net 7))
 (segment (start 139.18 107.85) (end 139.18 109.081) (width 0.3048) (layer F.Cu) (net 8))
 (segment (start 135.763 81.661) (end 135.72 81.618) (width 0.3048) (layer B.Cu) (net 8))
 (via (at 135.763 81.661) (size 0.6) (drill 0.4) (layers F.Cu B.Cu) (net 8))
 (segment (start 137.541 83.439) (end 135.763 81.661) (width 0.3048) (layer F.Cu) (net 8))
 (segment (start 143.51 83.439) (end 137.541 83.439) (width 0.3048) (layer F.Cu) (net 8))
 (segment (start 144.78 84.709) (end 143.51 83.439) (width 0.3048) (layer F.Cu) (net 8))
 (segment (start 144.78 106.299) (end 144.78 84.709) (width 0.3048) (layer F.Cu) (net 8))
 (segment (start 141.732 109.347) (end 144.78 106.299) (width 0.3048) (layer F.Cu) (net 8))
 (segment (start 139.446 109.347) (end 141.732 109.347) (width 0.3048) (layer F.Cu) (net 8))
 (segment (start 139.18 109.081) (end 139.446 109.347) (width 0.3048) (layer F.Cu) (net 8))
 (segment (start 135.72 81.618) (end 135.72 81.56) (width 0.3048) (layer B.Cu) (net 8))
 (segment (start 133.18 79.02) (end 133.18 79.037) (width 0.3048) (layer B.Cu) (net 9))
 (segment (start 133.18 79.037) (end 130.429 80.264) (width 0.3048) (layer B.Cu) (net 9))
 (segment (start 136.78 96.775) (end 136.78 99.35) (width 0.3048) (layer F.Cu) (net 9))
 (segment (start 130.429 90.424) (end 136.78 96.775) (width 0.3048) (layer F.Cu) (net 9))
 (via (at 130.429 90.424) (size 0.6) (drill 0.4) (layers F.Cu B.Cu) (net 9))
 (segment (start 130.429 80.264) (end 130.429 90.424) (width 0.3048) (layer B.Cu) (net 9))
 (segment (start 132.816 79.02) (end 133.18 79.02) (width 0.3048) (layer B.Cu) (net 9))
 (segment (start 133.122 79.02) (end 133.18 79.02) (width 0.3048) (layer B.Cu) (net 9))
 (segment (start 131.252 78.486) (end 132.969 78.486) (width 0.3048) (layer F.Cu) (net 10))
 (segment (start 138.26 76.751) (end 138.26 75.6) (width 0.3048) (layer F.Cu) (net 10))
 (segment (start 136.521802 78.486) (end 138.26 76.751) (width 0.3048) (layer F.Cu) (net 10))
 (segment (start 132.965802 78.486) (end 136.521802 78.486) (width 0.3048) (layer F.Cu) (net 10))
 (segment (start 132.969 78.486) (end 132.965802 78.486) (width 0.3048) (layer F.Cu) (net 10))
 (segment (start 134.62 92.426) (end 133.955 92.426) (width 0.3048) (layer F.Cu) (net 10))
 (segment (start 130.302 79.121) (end 130.937 78.486) (width 0.3048) (layer F.Cu) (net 10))
 (segment (start 130.302 88.773) (end 130.302 79.121) (width 0.3048) (layer F.Cu) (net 10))
 (segment (start 133.955 92.426) (end 130.302 88.773) (width 0.3048) (layer F.Cu) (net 10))
 (segment (start 130.937 78.486) (end 131.252 78.486) (width 0.3048) (layer F.Cu) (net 10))
 (segment (start 136.085 92.426) (end 134.62 92.426) (width 0.3048) (layer F.Cu) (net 10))
 (segment (start 134.62 92.426) (end 134.59 92.426) (width 0.3048) (layer F.Cu) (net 10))
 (segment (start 137.58 99.35) (end 137.58 95.416) (width 0.3048) (layer F.Cu) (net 10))
 (segment (start 136.085 93.921) (end 136.085 92.426) (width 0.3048) (layer F.Cu) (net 10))
 (segment (start 137.58 95.416) (end 136.085 93.921) (width 0.3048) (layer F.Cu) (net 10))
 (segment (start 134.239 91.176) (end 134.229 91.176) (width 0.3048) (layer F.Cu) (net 11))
 (segment (start 134.229 91.176) (end 131.252 88.199) (width 0.3048) (layer F.Cu) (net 11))
 (segment (start 131.252 88.199) (end 131.252 80.645) (width 0.3048) (layer F.Cu) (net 11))
 (segment (start 131.252 80.645) (end 131.572 80.645) (width 0.3048) (layer F.Cu) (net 11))
 (segment (start 131.572 80.645) (end 132.842 79.375) (width 0.3048) (layer F.Cu) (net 11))
 (segment (start 140.8 76.624) (end 140.8 75.6) (width 0.3048) (layer F.Cu) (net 11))
 (segment (start 138.049 79.375) (end 140.8 76.624) (width 0.3048) (layer F.Cu) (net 11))
 (segment (start 132.842 79.375) (end 138.049 79.375) (width 0.3048) (layer F.Cu) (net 11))
 (segment (start 136.085 91.176) (end 134.239 91.176) (width 0.3048) (layer F.Cu) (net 11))
 (segment (start 140.843 75.643) (end 140.8 75.6) (width 0.3048) (layer F.Cu) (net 11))
 (segment (start 138.38 99.35) (end 138.38 94.946) (width 0.3048) (layer F.Cu) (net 11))
 (segment (start 136.642 91.176) (end 136.085 91.176) (width 0.3048) (layer F.Cu) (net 11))
 (segment (start 137.16 91.694) (end 136.642 91.176) (width 0.3048) (layer F.Cu) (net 11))
 (segment (start 137.16 93.726) (end 137.16 91.694) (width 0.3048) (layer F.Cu) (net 11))
 (segment (start 138.38 94.946) (end 137.16 93.726) (width 0.3048) (layer F.Cu) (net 11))
 (segment (start 132.93 100.8) (end 132.169 100.8) (width 0.3048) (layer F.Cu) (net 13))
 (segment (start 132.169 100.8) (end 131.191 99.822) (width 0.3048) (layer F.Cu) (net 13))
 (segment (start 131.191 99.822) (end 131.191 93.345) (width 0.3048) (layer F.Cu) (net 13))
 (segment (start 131.191 93.345) (end 130.429 92.583) (width 0.3048) (layer F.Cu) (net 13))
 (segment (start 130.429 92.583) (end 130.429 91.694) (width 0.3048) (layer F.Cu) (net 13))
 (via (at 130.429 91.694) (size 0.6) (drill 0.4) (layers F.Cu B.Cu) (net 13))
 (segment (start 130.429 91.694) (end 132.207 89.916) (width 0.3048) (layer B.Cu) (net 13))
 (segment (start 132.207 89.916) (end 132.207 87.376) (width 0.3048) (layer B.Cu) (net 13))
 (via (at 132.207 87.376) (size 0.6) (drill 0.4) (layers F.Cu B.Cu) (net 13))
 (segment (start 132.207 87.376) (end 132.715 86.868) (width 0.3048) (layer F.Cu) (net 13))
 (segment (start 132.715 86.868) (end 135.509 86.868) (width 0.3048) (layer F.Cu) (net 13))
 (segment (start 135.509 86.868) (end 136.085 87.444) (width 0.3048) (layer F.Cu) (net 13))
 (segment (start 136.085 87.444) (end 136.085 88.676) (width 0.3048) (layer F.Cu) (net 13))
 (segment (start 134.38 99.35) (end 132.624 99.35) (width 0.3048) (layer F.Cu) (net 32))
 (segment (start 134.757 89.926) (end 136.085 89.926) (width 0.3048) (layer F.Cu) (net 32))
 (segment (start 133.096 88.265) (end 134.757 89.926) (width 0.3048) (layer F.Cu) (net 32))
 (via (at 133.096 88.265) (size 0.6) (drill 0.4) (layers F.Cu B.Cu) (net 32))
 (segment (start 133.096 90.551) (end 133.096 88.265) (width 0.3048) (layer B.Cu) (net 32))
 (segment (start 131.318 92.329) (end 133.096 90.551) (width 0.3048) (layer B.Cu) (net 32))
 (via (at 131.318 92.329) (size 0.6) (drill 0.4) (layers F.Cu B.Cu) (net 32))
 (segment (start 131.826 92.837) (end 131.318 92.329) (width 0.3048) (layer F.Cu) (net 32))
 (segment (start 131.826 98.552) (end 131.826 92.837) (width 0.3048) (layer F.Cu) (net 32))
 (segment (start 132.624 99.35) (end 131.826 98.552) (width 0.3048) (layer F.Cu) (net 32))
 (segment (start 136.085 89.926) (end 134.737 89.926) (width 0.3048) (layer F.Cu) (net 32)))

